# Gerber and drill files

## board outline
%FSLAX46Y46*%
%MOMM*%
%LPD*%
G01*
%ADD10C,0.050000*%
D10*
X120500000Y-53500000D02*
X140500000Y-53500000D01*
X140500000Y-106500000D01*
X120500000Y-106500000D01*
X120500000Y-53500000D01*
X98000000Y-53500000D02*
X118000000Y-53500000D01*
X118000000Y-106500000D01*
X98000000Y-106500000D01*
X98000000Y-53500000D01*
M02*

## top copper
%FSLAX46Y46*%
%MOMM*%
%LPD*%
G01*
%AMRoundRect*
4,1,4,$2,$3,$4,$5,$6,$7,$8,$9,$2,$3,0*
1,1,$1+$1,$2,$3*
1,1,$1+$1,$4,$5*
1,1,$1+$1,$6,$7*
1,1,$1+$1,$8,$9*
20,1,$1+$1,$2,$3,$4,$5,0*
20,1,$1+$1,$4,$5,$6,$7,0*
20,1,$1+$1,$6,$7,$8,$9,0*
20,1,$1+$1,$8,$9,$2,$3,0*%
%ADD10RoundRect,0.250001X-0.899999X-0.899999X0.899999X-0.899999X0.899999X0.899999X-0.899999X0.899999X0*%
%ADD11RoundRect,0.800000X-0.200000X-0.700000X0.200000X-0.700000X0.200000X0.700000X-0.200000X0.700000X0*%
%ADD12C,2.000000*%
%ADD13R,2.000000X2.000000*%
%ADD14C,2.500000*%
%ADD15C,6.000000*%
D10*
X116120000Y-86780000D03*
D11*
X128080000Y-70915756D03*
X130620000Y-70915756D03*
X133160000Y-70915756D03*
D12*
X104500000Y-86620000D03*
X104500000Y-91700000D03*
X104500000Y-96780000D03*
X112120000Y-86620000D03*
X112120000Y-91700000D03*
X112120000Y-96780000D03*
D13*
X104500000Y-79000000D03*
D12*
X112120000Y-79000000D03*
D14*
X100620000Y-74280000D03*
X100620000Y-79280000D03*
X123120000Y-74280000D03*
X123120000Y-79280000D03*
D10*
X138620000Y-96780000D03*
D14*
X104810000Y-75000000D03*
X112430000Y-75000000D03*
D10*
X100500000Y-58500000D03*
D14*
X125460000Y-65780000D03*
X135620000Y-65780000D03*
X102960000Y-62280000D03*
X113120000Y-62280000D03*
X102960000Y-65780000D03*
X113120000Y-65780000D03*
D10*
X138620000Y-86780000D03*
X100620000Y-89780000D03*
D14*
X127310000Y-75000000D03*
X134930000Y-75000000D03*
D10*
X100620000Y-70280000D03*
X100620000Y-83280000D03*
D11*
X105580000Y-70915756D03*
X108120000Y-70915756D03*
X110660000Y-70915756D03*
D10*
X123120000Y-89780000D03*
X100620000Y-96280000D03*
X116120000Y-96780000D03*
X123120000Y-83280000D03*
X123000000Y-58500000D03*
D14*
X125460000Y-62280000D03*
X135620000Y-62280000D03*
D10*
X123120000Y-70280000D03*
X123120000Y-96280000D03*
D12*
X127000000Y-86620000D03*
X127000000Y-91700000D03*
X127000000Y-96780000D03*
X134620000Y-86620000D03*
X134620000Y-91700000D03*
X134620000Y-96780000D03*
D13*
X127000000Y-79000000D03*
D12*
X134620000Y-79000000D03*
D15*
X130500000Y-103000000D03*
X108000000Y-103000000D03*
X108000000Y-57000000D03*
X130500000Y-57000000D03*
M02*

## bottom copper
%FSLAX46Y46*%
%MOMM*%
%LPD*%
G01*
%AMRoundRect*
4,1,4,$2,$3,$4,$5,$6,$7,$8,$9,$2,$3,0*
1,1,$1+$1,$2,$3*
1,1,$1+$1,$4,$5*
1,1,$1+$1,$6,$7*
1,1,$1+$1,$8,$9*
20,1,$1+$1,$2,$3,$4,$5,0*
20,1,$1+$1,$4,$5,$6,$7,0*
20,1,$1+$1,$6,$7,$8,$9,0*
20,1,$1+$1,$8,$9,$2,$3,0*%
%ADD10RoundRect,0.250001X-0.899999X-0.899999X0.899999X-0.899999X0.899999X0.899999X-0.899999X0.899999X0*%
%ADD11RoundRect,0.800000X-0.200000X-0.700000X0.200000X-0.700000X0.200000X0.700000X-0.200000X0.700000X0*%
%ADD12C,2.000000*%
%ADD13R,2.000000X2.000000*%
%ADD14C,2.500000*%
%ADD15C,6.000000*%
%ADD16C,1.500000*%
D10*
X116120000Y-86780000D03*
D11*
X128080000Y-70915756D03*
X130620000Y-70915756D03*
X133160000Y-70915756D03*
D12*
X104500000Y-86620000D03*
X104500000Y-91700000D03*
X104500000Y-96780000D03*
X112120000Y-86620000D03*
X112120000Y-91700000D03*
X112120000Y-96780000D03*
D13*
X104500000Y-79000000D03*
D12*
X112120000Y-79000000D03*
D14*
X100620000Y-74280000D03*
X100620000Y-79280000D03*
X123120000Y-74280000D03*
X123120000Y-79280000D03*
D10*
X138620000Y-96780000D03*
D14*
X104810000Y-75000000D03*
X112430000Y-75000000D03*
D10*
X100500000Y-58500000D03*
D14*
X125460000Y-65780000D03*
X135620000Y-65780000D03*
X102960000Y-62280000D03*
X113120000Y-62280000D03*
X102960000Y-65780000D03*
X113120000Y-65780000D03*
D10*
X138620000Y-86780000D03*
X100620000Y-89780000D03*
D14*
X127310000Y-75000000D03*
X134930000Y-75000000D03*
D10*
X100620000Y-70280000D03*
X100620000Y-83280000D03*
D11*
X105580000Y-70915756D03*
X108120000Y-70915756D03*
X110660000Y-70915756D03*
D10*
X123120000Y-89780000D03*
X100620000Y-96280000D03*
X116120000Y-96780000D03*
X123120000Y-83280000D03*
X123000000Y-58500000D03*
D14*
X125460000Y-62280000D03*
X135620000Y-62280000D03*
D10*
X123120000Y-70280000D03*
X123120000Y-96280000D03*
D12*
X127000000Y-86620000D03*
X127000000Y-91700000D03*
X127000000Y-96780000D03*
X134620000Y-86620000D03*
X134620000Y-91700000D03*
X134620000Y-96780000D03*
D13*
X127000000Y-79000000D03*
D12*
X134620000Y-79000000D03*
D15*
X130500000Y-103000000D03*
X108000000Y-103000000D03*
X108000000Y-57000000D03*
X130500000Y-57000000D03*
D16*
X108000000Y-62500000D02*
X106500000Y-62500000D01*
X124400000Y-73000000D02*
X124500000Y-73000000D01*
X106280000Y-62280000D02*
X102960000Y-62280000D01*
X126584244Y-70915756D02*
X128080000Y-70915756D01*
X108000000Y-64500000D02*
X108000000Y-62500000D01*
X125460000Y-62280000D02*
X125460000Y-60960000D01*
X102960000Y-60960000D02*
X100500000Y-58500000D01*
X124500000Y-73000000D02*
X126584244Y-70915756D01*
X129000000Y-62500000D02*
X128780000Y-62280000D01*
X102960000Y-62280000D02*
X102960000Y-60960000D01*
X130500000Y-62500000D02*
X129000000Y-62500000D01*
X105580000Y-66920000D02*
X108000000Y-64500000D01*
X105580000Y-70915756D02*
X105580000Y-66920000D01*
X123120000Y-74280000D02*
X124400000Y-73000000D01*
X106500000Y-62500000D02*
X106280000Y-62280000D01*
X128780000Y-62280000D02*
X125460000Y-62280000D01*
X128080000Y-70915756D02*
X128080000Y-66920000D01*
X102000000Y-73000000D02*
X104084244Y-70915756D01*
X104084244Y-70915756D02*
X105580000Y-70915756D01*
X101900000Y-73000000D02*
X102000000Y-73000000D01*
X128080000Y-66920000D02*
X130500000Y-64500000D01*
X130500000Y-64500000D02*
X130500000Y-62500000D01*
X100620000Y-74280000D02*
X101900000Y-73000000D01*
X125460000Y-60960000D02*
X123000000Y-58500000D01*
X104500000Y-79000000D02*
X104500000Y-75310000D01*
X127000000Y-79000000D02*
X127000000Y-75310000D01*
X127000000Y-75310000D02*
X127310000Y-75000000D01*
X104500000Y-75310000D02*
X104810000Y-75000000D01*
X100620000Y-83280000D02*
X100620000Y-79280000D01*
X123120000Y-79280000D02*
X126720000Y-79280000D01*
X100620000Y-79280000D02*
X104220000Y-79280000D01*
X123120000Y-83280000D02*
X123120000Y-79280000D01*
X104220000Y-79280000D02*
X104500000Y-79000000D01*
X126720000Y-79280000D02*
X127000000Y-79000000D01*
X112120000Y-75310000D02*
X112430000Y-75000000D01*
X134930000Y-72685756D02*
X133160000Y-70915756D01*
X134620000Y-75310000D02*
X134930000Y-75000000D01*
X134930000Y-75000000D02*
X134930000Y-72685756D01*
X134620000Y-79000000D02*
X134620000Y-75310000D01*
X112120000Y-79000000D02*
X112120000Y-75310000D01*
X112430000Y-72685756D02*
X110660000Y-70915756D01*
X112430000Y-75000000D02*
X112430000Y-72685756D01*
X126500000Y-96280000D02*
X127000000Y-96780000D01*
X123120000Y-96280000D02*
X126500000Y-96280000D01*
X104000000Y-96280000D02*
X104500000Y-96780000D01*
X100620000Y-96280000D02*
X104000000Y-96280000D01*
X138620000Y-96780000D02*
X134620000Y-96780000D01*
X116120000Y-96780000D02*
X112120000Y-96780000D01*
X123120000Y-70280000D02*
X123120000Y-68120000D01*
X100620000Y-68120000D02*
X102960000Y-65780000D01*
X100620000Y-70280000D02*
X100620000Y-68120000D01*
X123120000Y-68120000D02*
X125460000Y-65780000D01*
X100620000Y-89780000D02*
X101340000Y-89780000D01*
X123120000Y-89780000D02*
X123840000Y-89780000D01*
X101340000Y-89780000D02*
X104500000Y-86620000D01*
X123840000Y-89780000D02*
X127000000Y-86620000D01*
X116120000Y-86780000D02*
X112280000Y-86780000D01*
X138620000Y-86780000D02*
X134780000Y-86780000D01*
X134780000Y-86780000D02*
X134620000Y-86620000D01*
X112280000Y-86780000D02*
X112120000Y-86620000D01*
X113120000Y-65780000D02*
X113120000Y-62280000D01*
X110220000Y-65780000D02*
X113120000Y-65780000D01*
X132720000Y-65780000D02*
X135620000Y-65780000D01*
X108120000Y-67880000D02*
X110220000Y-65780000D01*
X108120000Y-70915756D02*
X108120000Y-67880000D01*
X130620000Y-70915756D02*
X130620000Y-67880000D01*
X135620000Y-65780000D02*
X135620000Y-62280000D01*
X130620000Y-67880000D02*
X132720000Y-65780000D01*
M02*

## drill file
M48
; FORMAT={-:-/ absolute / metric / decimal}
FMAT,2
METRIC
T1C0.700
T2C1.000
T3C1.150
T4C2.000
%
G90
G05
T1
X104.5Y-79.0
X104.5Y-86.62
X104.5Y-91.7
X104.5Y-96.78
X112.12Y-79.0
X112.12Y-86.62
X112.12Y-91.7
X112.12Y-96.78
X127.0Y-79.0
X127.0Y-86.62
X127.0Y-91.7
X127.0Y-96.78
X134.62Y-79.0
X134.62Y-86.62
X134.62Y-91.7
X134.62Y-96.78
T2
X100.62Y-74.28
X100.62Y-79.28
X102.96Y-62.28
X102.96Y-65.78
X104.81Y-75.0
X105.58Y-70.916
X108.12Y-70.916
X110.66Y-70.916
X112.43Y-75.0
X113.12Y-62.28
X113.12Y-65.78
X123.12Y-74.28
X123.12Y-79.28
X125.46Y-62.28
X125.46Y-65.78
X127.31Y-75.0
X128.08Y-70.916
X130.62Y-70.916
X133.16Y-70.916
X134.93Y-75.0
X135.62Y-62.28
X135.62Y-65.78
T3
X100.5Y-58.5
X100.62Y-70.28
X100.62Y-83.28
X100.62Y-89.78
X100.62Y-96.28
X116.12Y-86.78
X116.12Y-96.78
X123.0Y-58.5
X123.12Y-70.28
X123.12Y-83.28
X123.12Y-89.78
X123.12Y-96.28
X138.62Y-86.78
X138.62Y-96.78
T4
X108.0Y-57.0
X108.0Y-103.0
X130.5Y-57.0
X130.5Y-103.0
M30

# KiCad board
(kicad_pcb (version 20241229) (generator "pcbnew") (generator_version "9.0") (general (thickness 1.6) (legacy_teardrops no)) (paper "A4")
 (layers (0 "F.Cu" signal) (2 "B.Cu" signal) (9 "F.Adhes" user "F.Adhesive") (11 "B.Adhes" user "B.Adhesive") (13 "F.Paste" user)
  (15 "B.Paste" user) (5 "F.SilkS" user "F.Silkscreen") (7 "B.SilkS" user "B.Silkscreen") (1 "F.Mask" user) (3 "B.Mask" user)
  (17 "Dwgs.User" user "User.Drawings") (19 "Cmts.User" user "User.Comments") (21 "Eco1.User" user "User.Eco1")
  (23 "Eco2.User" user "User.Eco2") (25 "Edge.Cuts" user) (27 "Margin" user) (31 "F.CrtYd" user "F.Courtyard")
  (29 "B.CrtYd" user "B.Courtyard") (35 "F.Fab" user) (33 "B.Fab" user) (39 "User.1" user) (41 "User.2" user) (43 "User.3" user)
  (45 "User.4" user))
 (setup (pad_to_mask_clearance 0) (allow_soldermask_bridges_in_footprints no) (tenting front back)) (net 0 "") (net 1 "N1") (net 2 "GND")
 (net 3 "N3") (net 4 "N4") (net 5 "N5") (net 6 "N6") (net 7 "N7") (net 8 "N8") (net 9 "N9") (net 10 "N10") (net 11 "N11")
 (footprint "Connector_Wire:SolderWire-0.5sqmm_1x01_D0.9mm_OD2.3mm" (layer "F.Cu") (at 116.12 86.78)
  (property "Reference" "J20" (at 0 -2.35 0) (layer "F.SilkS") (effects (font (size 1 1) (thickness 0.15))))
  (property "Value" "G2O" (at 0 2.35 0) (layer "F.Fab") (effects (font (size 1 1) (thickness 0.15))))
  (pad "1" thru_hole roundrect (at 0 0) (size 2.3 2.3) (drill 1.15) (layers "*.Cu" "*.Mask") (remove_unused_layers no)
   (roundrect_rratio 0.108696) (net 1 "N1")))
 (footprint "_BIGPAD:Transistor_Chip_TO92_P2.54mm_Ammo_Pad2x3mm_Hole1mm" (layer "F.Cu") (at 128.08 70.915756)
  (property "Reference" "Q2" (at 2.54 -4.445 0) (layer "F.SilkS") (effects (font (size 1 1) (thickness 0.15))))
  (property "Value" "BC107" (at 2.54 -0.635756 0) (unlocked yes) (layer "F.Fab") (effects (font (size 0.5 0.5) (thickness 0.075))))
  (pad "1" thru_hole roundrect (at 0 0) (size 2 3) (drill 1) (layers "*.Cu" "*.Mask") (remove_unused_layers no) (roundrect_rratio 0.4)
   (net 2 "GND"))
  (pad "2" thru_hole roundrect (at 2.54 0) (size 2 3) (drill 1) (layers "*.Cu" "*.Mask") (remove_unused_layers no) (roundrect_rratio 0.4)
   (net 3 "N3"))
  (pad "3" thru_hole roundrect (at 5.08 0) (size 2 3) (drill 1) (layers "*.Cu" "*.Mask") (remove_unused_layers no) (roundrect_rratio 0.4)
   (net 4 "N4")))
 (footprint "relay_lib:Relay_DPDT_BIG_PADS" (layer "F.Cu") (at 104.5 79)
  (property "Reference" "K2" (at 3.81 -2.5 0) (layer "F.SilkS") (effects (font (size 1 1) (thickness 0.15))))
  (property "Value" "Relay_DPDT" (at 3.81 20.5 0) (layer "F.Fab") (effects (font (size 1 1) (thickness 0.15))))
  (pad "11" thru_hole circle (at 0 7.62) (size 2 2) (drill 0.7) (layers "*.Cu" "*.Mask") (remove_unused_layers no) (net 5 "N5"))
  (pad "12" thru_hole circle (at 0 12.7) (size 2 2) (drill 0.7) (layers "*.Cu" "*.Mask") (remove_unused_layers no) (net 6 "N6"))
  (pad "14" thru_hole circle (at 0 17.78) (size 2 2) (drill 0.7) (layers "*.Cu" "*.Mask") (remove_unused_layers no) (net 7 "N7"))
  (pad "21" thru_hole circle (at 7.62 7.62) (size 2 2) (drill 0.7) (layers "*.Cu" "*.Mask") (remove_unused_layers no) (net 1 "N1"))
  (pad "22" thru_hole circle (at 7.62 12.7) (size 2 2) (drill 0.7) (layers "*.Cu" "*.Mask") (remove_unused_layers no) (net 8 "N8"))
  (pad "24" thru_hole circle (at 7.62 17.78) (size 2 2) (drill 0.7) (layers "*.Cu" "*.Mask") (remove_unused_layers no) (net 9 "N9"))
  (pad "A1" thru_hole rect (at 0 0) (size 2 2) (drill 0.7) (layers "*.Cu" "*.Mask") (remove_unused_layers no) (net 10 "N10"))
  (pad "A2" thru_hole circle (at 7.62 0) (size 2 2) (drill 0.7) (layers "*.Cu" "*.Mask") (remove_unused_layers no) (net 4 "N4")))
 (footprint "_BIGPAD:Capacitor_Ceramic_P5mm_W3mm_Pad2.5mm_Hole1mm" (layer "F.Cu") (at 100.62 74.28 -90)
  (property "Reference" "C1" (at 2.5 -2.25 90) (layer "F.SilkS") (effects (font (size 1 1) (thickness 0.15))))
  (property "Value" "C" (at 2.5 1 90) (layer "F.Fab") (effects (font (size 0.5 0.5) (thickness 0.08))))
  (pad "1" thru_hole circle (at 0 0) (size 2.5 2.5) (drill 1) (layers "*.Cu" "*.Mask") (remove_unused_layers no) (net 2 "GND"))
  (pad "2" thru_hole circle (at 5 0) (size 2.5 2.5) (drill 1) (layers "*.Cu" "*.Mask") (remove_unused_layers no) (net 10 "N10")))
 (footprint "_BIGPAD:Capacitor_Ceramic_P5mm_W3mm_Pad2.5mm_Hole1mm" (layer "F.Cu") (at 123.12 74.28 -90)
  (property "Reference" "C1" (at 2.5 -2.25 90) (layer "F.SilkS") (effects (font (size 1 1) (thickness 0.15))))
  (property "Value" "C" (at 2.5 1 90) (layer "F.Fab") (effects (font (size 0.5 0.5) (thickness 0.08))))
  (pad "1" thru_hole circle (at 0 0) (size 2.5 2.5) (drill 1) (layers "*.Cu" "*.Mask") (remove_unused_layers no) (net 2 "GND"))
  (pad "2" thru_hole circle (at 5 0) (size 2.5 2.5) (drill 1) (layers "*.Cu" "*.Mask") (remove_unused_layers no) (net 10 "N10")))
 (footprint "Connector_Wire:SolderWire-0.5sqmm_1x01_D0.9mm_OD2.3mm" (layer "F.Cu") (at 138.62 96.78)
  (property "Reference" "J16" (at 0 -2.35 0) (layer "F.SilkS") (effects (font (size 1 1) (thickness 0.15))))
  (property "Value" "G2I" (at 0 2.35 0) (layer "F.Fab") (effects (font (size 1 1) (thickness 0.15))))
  (pad "1" thru_hole roundrect (at 0 0) (size 2.3 2.3) (drill 1.15) (layers "*.Cu" "*.Mask") (remove_unused_layers no)
   (roundrect_rratio 0.108696) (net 9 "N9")))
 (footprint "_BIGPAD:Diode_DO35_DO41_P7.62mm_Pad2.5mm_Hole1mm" (layer "F.Cu") (at 104.81 75)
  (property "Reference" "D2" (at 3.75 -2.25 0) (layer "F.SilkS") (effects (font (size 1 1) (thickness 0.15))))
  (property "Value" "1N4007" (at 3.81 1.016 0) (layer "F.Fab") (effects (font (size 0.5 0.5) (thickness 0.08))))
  (pad "1" thru_hole circle (at 0 0 90) (size 2.5 2.5) (drill 1) (layers "*.Cu" "*.Mask") (remove_unused_layers no) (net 10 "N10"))
  (pad "2" thru_hole circle (at 7.62 0 90) (size 2.5 2.5) (drill 1) (layers "*.Cu" "*.Mask") (remove_unused_layers no) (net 4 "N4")))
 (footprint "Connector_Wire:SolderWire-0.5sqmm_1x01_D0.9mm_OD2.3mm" (layer "F.Cu") (at 100.5 58.5)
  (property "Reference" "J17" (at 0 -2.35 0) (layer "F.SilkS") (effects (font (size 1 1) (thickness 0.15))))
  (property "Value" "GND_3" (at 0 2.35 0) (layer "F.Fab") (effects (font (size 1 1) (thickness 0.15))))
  (pad "1" thru_hole roundrect (at 0 0) (size 2.3 2.3) (drill 1.15) (layers "*.Cu" "*.Mask") (remove_unused_layers no)
   (roundrect_rratio 0.108696) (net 2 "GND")))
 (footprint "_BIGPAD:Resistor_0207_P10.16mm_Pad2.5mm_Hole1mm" (layer "F.Cu") (at 125.46 65.78)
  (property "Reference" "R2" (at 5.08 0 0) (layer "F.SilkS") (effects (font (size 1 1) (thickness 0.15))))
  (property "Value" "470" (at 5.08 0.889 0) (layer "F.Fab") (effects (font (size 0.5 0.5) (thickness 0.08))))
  (pad "1" thru_hole circle (at 0 0 90) (size 2.5 2.5) (drill 1) (layers "*.Cu" "*.Mask") (remove_unused_layers no) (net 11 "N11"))
  (pad "2" thru_hole circle (at 10.16 0 90) (size 2.5 2.5) (drill 1) (layers "*.Cu" "*.Mask") (remove_unused_layers no) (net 3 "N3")))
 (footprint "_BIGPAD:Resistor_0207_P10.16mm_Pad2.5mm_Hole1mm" (layer "F.Cu") (at 102.96 62.28)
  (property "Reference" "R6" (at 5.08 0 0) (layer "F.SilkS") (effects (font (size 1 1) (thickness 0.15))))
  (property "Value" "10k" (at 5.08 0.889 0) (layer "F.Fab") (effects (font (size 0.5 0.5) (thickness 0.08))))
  (pad "1" thru_hole circle (at 0 0 90) (size 2.5 2.5) (drill 1) (layers "*.Cu" "*.Mask") (remove_unused_layers no) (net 2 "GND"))
  (pad "2" thru_hole circle (at 10.16 0 90) (size 2.5 2.5) (drill 1) (layers "*.Cu" "*.Mask") (remove_unused_layers no) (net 3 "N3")))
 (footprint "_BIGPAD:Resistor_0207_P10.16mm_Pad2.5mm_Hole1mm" (layer "F.Cu") (at 102.96 65.78)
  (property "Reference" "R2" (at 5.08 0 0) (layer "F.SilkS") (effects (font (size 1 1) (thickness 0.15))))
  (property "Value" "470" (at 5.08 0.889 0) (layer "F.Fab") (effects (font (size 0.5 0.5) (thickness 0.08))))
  (pad "1" thru_hole circle (at 0 0 90) (size 2.5 2.5) (drill 1) (layers "*.Cu" "*.Mask") (remove_unused_layers no) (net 11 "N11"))
  (pad "2" thru_hole circle (at 10.16 0 90) (size 2.5 2.5) (drill 1) (layers "*.Cu" "*.Mask") (remove_unused_layers no) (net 3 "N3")))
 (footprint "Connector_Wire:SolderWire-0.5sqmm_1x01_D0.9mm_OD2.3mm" (layer "F.Cu") (at 138.62 86.78)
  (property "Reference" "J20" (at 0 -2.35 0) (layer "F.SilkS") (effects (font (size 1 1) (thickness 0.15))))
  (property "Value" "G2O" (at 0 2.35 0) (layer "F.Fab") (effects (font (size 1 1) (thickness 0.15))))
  (pad "1" thru_hole roundrect (at 0 0) (size 2.3 2.3) (drill 1.15) (layers "*.Cu" "*.Mask") (remove_unused_layers no)
   (roundrect_rratio 0.108696) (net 1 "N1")))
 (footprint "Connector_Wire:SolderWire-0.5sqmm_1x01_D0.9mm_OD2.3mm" (layer "F.Cu") (at 100.62 89.78)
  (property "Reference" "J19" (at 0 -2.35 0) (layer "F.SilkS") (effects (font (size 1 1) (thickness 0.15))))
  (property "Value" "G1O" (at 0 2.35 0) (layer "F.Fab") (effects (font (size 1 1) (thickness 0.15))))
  (pad "1" thru_hole roundrect (at 0 0) (size 2.3 2.3) (drill 1.15) (layers "*.Cu" "*.Mask") (remove_unused_layers no)
   (roundrect_rratio 0.108696) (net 5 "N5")))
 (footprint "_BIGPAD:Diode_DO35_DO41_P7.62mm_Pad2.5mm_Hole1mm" (layer "F.Cu") (at 127.31 75)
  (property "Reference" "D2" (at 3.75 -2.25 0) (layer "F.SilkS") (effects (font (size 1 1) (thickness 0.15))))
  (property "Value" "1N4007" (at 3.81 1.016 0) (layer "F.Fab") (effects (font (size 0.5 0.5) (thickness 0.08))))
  (pad "1" thru_hole circle (at 0 0 90) (size 2.5 2.5) (drill 1) (layers "*.Cu" "*.Mask") (remove_unused_layers no) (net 10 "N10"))
  (pad "2" thru_hole circle (at 7.62 0 90) (size 2.5 2.5) (drill 1) (layers "*.Cu" "*.Mask") (remove_unused_layers no) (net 4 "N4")))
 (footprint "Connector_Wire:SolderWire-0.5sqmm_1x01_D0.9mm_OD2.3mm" (layer "F.Cu") (at 100.62 70.28)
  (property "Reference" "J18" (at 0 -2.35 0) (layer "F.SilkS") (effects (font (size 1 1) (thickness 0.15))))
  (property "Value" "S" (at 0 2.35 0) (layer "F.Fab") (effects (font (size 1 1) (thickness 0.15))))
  (pad "1" thru_hole roundrect (at 0 0) (size 2.3 2.3) (drill 1.15) (layers "*.Cu" "*.Mask") (remove_unused_layers no)
   (roundrect_rratio 0.108696) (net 11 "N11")))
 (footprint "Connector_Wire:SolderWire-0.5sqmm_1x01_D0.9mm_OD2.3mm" (layer "F.Cu") (at 100.62 83.28)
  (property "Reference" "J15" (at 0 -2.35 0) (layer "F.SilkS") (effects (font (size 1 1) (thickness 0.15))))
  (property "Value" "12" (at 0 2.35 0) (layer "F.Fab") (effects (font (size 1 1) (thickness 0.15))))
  (pad "1" thru_hole roundrect (at 0 0) (size 2.3 2.3) (drill 1.15) (layers "*.Cu" "*.Mask") (remove_unused_layers no)
   (roundrect_rratio 0.108696) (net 10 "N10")))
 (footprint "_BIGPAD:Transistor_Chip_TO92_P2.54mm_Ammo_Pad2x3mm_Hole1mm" (layer "F.Cu") (at 105.58 70.915756)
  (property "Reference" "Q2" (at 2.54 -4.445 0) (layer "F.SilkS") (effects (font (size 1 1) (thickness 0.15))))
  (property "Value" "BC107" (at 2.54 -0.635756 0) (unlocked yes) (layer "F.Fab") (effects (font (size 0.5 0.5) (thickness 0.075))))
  (pad "1" thru_hole roundrect (at 0 0) (size 2 3) (drill 1) (layers "*.Cu" "*.Mask") (remove_unused_layers no) (roundrect_rratio 0.4)
   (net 2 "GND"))
  (pad "2" thru_hole roundrect (at 2.54 0) (size 2 3) (drill 1) (layers "*.Cu" "*.Mask") (remove_unused_layers no) (roundrect_rratio 0.4)
   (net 3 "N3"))
  (pad "3" thru_hole roundrect (at 5.08 0) (size 2 3) (drill 1) (layers "*.Cu" "*.Mask") (remove_unused_layers no) (roundrect_rratio 0.4)
   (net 4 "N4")))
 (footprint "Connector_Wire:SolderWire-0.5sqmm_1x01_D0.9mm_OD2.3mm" (layer "F.Cu") (at 123.12 89.78)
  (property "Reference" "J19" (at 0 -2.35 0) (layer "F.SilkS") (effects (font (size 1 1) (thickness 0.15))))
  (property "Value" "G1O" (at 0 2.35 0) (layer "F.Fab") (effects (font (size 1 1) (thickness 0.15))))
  (pad "1" thru_hole roundrect (at 0 0) (size 2.3 2.3) (drill 1.15) (layers "*.Cu" "*.Mask") (remove_unused_layers no)
   (roundrect_rratio 0.108696) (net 5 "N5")))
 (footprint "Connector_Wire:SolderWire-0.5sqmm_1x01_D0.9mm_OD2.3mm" (layer "F.Cu") (at 100.62 96.28)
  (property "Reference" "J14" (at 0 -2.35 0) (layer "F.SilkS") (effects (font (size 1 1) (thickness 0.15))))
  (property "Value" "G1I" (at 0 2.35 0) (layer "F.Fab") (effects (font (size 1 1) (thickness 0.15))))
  (pad "1" thru_hole roundrect (at 0 0) (size 2.3 2.3) (drill 1.15) (layers "*.Cu" "*.Mask") (remove_unused_layers no)
   (roundrect_rratio 0.108696) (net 7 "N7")))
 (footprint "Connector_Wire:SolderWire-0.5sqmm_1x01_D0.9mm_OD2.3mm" (layer "F.Cu") (at 116.12 96.78)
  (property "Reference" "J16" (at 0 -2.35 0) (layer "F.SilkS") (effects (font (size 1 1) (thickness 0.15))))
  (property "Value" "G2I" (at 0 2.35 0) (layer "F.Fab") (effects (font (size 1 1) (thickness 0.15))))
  (pad "1" thru_hole roundrect (at 0 0) (size 2.3 2.3) (drill 1.15) (layers "*.Cu" "*.Mask") (remove_unused_layers no)
   (roundrect_rratio 0.108696) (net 9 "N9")))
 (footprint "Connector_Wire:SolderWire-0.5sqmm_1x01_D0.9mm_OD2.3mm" (layer "F.Cu") (at 123.12 83.28)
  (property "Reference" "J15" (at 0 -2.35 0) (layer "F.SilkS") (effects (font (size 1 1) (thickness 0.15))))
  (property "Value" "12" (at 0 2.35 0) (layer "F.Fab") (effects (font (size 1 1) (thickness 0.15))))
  (pad "1" thru_hole roundrect (at 0 0) (size 2.3 2.3) (drill 1.15) (layers "*.Cu" "*.Mask") (remove_unused_layers no)
   (roundrect_rratio 0.108696) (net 10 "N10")))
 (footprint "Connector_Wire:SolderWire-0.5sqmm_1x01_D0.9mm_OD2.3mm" (layer "F.Cu") (at 123 58.5)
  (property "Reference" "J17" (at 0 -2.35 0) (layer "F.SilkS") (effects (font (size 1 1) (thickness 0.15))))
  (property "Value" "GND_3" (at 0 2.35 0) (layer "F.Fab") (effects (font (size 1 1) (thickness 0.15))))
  (pad "1" thru_hole roundrect (at 0 0) (size 2.3 2.3) (drill 1.15) (layers "*.Cu" "*.Mask") (remove_unused_layers no)
   (roundrect_rratio 0.108696) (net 2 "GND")))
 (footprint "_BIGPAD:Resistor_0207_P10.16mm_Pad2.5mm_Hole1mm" (layer "F.Cu") (at 125.46 62.28)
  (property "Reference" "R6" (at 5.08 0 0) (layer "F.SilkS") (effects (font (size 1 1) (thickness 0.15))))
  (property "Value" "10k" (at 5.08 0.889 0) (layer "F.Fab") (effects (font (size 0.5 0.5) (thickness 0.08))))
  (pad "1" thru_hole circle (at 0 0 90) (size 2.5 2.5) (drill 1) (layers "*.Cu" "*.Mask") (remove_unused_layers no) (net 2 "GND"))
  (pad "2" thru_hole circle (at 10.16 0 90) (size 2.5 2.5) (drill 1) (layers "*.Cu" "*.Mask") (remove_unused_layers no) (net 3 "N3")))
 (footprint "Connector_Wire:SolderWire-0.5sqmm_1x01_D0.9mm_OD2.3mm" (layer "F.Cu") (at 123.12 70.28)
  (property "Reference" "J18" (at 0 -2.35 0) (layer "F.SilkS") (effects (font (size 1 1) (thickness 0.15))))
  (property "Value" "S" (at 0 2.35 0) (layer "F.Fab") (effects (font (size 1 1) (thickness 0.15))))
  (pad "1" thru_hole roundrect (at 0 0) (size 2.3 2.3) (drill 1.15) (layers "*.Cu" "*.Mask") (remove_unused_layers no)
   (roundrect_rratio 0.108696) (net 11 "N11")))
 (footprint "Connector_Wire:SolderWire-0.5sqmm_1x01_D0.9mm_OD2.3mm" (layer "F.Cu") (at 123.12 96.28)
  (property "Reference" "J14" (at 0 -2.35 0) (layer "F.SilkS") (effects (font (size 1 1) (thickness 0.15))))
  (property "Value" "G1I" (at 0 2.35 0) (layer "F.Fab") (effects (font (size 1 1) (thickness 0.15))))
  (pad "1" thru_hole roundrect (at 0 0) (size 2.3 2.3) (drill 1.15) (layers "*.Cu" "*.Mask") (remove_unused_layers no)
   (roundrect_rratio 0.108696) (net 7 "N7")))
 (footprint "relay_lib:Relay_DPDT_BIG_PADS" (layer "F.Cu") (at 127 79)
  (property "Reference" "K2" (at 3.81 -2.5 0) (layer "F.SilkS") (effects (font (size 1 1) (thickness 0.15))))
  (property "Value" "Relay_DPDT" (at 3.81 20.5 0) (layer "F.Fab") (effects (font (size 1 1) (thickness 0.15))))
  (pad "11" thru_hole circle (at 0 7.62) (size 2 2) (drill 0.7) (layers "*.Cu" "*.Mask") (remove_unused_layers no) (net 5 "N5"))
  (pad "12" thru_hole circle (at 0 12.7) (size 2 2) (drill 0.7) (layers "*.Cu" "*.Mask") (remove_unused_layers no) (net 6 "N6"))
  (pad "14" thru_hole circle (at 0 17.78) (size 2 2) (drill 0.7) (layers "*.Cu" "*.Mask") (remove_unused_layers no) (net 7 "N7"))
  (pad "21" thru_hole circle (at 7.62 7.62) (size 2 2) (drill 0.7) (layers "*.Cu" "*.Mask") (remove_unused_layers no) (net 1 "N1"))
  (pad "22" thru_hole circle (at 7.62 12.7) (size 2 2) (drill 0.7) (layers "*.Cu" "*.Mask") (remove_unused_layers no) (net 8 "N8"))
  (pad "24" thru_hole circle (at 7.62 17.78) (size 2 2) (drill 0.7) (layers "*.Cu" "*.Mask") (remove_unused_layers no) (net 9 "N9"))
  (pad "A1" thru_hole rect (at 0 0) (size 2 2) (drill 0.7) (layers "*.Cu" "*.Mask") (remove_unused_layers no) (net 10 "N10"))
  (pad "A2" thru_hole circle (at 7.62 0) (size 2 2) (drill 0.7) (layers "*.Cu" "*.Mask") (remove_unused_layers no) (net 4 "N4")))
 (gr_rect (start 120.5 53.5) (end 140.5 106.5) (stroke (width 0.05) (type default)) (fill no) (layer "Edge.Cuts"))
 (gr_rect (start 98 53.5) (end 118 106.5) (stroke (width 0.05) (type default)) (fill no) (layer "Edge.Cuts"))
 (via (at 130.5 103) (size 6) (drill 2) (layers "F.Cu" "B.Cu") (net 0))
 (via (at 108 103) (size 6) (drill 2) (layers "F.Cu" "B.Cu") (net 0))
 (via (at 108 57) (size 6) (drill 2) (layers "F.Cu" "B.Cu") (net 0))
 (via (at 130.5 57) (size 6) (drill 2) (layers "F.Cu" "B.Cu") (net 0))
 (segment (start 108 62.5) (end 106.5 62.5) (width 1.5) (layer "B.Cu") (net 2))
 (segment (start 124.4 73) (end 124.5 73) (width 1.5) (layer "B.Cu") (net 2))
 (segment (start 106.28 62.28) (end 102.96 62.28) (width 1.5) (layer "B.Cu") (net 2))
 (segment (start 126.584244 70.915756) (end 128.08 70.915756) (width 1.5) (layer "B.Cu") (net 2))
 (segment (start 108 64.5) (end 108 62.5) (width 1.5) (layer "B.Cu") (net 2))
 (segment (start 125.46 62.28) (end 125.46 60.96) (width 1.5) (layer "B.Cu") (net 2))
 (segment (start 102.96 60.96) (end 100.5 58.5) (width 1.5) (layer "B.Cu") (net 2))
 (segment (start 124.5 73) (end 126.584244 70.915756) (width 1.5) (layer "B.Cu") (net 2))
 (segment (start 129 62.5) (end 128.78 62.28) (width 1.5) (layer "B.Cu") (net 2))
 (segment (start 102.96 62.28) (end 102.96 60.96) (width 1.5) (layer "B.Cu") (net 2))
 (segment (start 130.5 62.5) (end 129 62.5) (width 1.5) (layer "B.Cu") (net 2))
 (segment (start 105.58 66.92) (end 108 64.5) (width 1.5) (layer "B.Cu") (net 2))
 (segment (start 105.58 70.915756) (end 105.58 66.92) (width 1.5) (layer "B.Cu") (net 2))
 (segment (start 123.12 74.28) (end 124.4 73) (width 1.5) (layer "B.Cu") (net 2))
 (segment (start 106.5 62.5) (end 106.28 62.28) (width 1.5) (layer "B.Cu") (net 2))
 (segment (start 128.78 62.28) (end 125.46 62.28) (width 1.5) (layer "B.Cu") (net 2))
 (segment (start 128.08 70.915756) (end 128.08 66.92) (width 1.5) (layer "B.Cu") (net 2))
 (segment (start 102 73) (end 104.084244 70.915756) (width 1.5) (layer "B.Cu") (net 2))
 (segment (start 104.084244 70.915756) (end 105.58 70.915756) (width 1.5) (layer "B.Cu") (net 2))
 (segment (start 101.9 73) (end 102 73) (width 1.5) (layer "B.Cu") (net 2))
 (segment (start 128.08 66.92) (end 130.5 64.5) (width 1.5) (layer "B.Cu") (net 2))
 (segment (start 130.5 64.5) (end 130.5 62.5) (width 1.5) (layer "B.Cu") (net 2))
 (segment (start 100.62 74.28) (end 101.9 73) (width 1.5) (layer "B.Cu") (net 2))
 (segment (start 125.46 60.96) (end 123 58.5) (width 1.5) (layer "B.Cu") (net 2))
 (segment (start 104.5 79) (end 104.5 75.31) (width 1.5) (layer "B.Cu") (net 10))
 (segment (start 127 79) (end 127 75.31) (width 1.5) (layer "B.Cu") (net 10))
 (segment (start 127 75.31) (end 127.31 75) (width 1.5) (layer "B.Cu") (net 10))
 (segment (start 104.5 75.31) (end 104.81 75) (width 1.5) (layer "B.Cu") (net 10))
 (segment (start 100.62 83.28) (end 100.62 79.28) (width 1.5) (layer "B.Cu") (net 10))
 (segment (start 123.12 79.28) (end 126.72 79.28) (width 1.5) (layer "B.Cu") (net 10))
 (segment (start 100.62 79.28) (end 104.22 79.28) (width 1.5) (layer "B.Cu") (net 10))
 (segment (start 123.12 83.28) (end 123.12 79.28) (width 1.5) (layer "B.Cu") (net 10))
 (segment (start 104.22 79.28) (end 104.5 79) (width 1.5) (layer "B.Cu") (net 10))
 (segment (start 126.72 79.28) (end 127 79) (width 1.5) (layer "B.Cu") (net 10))
 (segment (start 112.12 75.31) (end 112.43 75) (width 1.5) (layer "B.Cu") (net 4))
 (segment (start 134.93 72.685756) (end 133.16 70.915756) (width 1.5) (layer "B.Cu") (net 4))
 (segment (start 134.62 75.31) (end 134.93 75) (width 1.5) (layer "B.Cu") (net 4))
 (segment (start 134.93 75) (end 134.93 72.685756) (width 1.5) (layer "B.Cu") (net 4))
 (segment (start 134.62 79) (end 134.62 75.31) (width 1.5) (layer "B.Cu") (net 4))
 (segment (start 112.12 79) (end 112.12 75.31) (width 1.5) (layer "B.Cu") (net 4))
 (segment (start 112.43 72.685756) (end 110.66 70.915756) (width 1.5) (layer "B.Cu") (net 4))
 (segment (start 112.43 75) (end 112.43 72.685756) (width 1.5) (layer "B.Cu") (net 4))
 (segment (start 126.5 96.28) (end 127 96.78) (width 1.5) (layer "B.Cu") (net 7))
 (segment (start 123.12 96.28) (end 126.5 96.28) (width 1.5) (layer "B.Cu") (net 7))
 (segment (start 104 96.28) (end 104.5 96.78) (width 1.5) (layer "B.Cu") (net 7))
 (segment (start 100.62 96.28) (end 104 96.28) (width 1.5) (layer "B.Cu") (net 7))
 (segment (start 138.62 96.78) (end 134.62 96.78) (width 1.5) (layer "B.Cu") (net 9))
 (segment (start 116.12 96.78) (end 112.12 96.78) (width 1.5) (layer "B.Cu") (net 9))
 (segment (start 123.12 70.28) (end 123.12 68.12) (width 1.5) (layer "B.Cu") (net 11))
 (segment (start 100.62 68.12) (end 102.96 65.78) (width 1.5) (layer "B.Cu") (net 11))
 (segment (start 100.62 70.28) (end 100.62 68.12) (width 1.5) (layer "B.Cu") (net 11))
 (segment (start 123.12 68.12) (end 125.46 65.78) (width 1.5) (layer "B.Cu") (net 11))
 (segment (start 100.62 89.78) (end 101.34 89.78) (width 1.5) (layer "B.Cu") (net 5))
 (segment (start 123.12 89.78) (end 123.84 89.78) (width 1.5) (layer "B.Cu") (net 5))
 (segment (start 101.34 89.78) (end 104.5 86.62) (width 1.5) (layer "B.Cu") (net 5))
 (segment (start 123.84 89.78) (end 127 86.62) (width 1.5) (layer "B.Cu") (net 5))
 (segment (start 116.12 86.78) (end 112.28 86.78) (width 1.5) (layer "B.Cu") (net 1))
 (segment (start 138.62 86.78) (end 134.78 86.78) (width 1.5) (layer "B.Cu") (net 1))
 (segment (start 134.78 86.78) (end 134.62 86.62) (width 1.5) (layer "B.Cu") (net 1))
 (segment (start 112.28 86.78) (end 112.12 86.62) (width 1.5) (layer "B.Cu") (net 1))
 (segment (start 113.12 65.78) (end 113.12 62.28) (width 1.5) (layer "B.Cu") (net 3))
 (segment (start 110.22 65.78) (end 113.12 65.78) (width 1.5) (layer "B.Cu") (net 3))
 (segment (start 132.72 65.78) (end 135.62 65.78) (width 1.5) (layer "B.Cu") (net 3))
 (segment (start 108.12 67.88) (end 110.22 65.78) (width 1.5) (layer "B.Cu") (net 3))
 (segment (start 108.12 70.915756) (end 108.12 67.88) (width 1.5) (layer "B.Cu") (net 3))
 (segment (start 130.62 70.915756) (end 130.62 67.88) (width 1.5) (layer "B.Cu") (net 3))
 (segment (start 135.62 65.78) (end 135.62 62.28) (width 1.5) (layer "B.Cu") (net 3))
 (segment (start 130.62 67.88) (end 132.72 65.78) (width 1.5) (layer "B.Cu") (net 3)))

